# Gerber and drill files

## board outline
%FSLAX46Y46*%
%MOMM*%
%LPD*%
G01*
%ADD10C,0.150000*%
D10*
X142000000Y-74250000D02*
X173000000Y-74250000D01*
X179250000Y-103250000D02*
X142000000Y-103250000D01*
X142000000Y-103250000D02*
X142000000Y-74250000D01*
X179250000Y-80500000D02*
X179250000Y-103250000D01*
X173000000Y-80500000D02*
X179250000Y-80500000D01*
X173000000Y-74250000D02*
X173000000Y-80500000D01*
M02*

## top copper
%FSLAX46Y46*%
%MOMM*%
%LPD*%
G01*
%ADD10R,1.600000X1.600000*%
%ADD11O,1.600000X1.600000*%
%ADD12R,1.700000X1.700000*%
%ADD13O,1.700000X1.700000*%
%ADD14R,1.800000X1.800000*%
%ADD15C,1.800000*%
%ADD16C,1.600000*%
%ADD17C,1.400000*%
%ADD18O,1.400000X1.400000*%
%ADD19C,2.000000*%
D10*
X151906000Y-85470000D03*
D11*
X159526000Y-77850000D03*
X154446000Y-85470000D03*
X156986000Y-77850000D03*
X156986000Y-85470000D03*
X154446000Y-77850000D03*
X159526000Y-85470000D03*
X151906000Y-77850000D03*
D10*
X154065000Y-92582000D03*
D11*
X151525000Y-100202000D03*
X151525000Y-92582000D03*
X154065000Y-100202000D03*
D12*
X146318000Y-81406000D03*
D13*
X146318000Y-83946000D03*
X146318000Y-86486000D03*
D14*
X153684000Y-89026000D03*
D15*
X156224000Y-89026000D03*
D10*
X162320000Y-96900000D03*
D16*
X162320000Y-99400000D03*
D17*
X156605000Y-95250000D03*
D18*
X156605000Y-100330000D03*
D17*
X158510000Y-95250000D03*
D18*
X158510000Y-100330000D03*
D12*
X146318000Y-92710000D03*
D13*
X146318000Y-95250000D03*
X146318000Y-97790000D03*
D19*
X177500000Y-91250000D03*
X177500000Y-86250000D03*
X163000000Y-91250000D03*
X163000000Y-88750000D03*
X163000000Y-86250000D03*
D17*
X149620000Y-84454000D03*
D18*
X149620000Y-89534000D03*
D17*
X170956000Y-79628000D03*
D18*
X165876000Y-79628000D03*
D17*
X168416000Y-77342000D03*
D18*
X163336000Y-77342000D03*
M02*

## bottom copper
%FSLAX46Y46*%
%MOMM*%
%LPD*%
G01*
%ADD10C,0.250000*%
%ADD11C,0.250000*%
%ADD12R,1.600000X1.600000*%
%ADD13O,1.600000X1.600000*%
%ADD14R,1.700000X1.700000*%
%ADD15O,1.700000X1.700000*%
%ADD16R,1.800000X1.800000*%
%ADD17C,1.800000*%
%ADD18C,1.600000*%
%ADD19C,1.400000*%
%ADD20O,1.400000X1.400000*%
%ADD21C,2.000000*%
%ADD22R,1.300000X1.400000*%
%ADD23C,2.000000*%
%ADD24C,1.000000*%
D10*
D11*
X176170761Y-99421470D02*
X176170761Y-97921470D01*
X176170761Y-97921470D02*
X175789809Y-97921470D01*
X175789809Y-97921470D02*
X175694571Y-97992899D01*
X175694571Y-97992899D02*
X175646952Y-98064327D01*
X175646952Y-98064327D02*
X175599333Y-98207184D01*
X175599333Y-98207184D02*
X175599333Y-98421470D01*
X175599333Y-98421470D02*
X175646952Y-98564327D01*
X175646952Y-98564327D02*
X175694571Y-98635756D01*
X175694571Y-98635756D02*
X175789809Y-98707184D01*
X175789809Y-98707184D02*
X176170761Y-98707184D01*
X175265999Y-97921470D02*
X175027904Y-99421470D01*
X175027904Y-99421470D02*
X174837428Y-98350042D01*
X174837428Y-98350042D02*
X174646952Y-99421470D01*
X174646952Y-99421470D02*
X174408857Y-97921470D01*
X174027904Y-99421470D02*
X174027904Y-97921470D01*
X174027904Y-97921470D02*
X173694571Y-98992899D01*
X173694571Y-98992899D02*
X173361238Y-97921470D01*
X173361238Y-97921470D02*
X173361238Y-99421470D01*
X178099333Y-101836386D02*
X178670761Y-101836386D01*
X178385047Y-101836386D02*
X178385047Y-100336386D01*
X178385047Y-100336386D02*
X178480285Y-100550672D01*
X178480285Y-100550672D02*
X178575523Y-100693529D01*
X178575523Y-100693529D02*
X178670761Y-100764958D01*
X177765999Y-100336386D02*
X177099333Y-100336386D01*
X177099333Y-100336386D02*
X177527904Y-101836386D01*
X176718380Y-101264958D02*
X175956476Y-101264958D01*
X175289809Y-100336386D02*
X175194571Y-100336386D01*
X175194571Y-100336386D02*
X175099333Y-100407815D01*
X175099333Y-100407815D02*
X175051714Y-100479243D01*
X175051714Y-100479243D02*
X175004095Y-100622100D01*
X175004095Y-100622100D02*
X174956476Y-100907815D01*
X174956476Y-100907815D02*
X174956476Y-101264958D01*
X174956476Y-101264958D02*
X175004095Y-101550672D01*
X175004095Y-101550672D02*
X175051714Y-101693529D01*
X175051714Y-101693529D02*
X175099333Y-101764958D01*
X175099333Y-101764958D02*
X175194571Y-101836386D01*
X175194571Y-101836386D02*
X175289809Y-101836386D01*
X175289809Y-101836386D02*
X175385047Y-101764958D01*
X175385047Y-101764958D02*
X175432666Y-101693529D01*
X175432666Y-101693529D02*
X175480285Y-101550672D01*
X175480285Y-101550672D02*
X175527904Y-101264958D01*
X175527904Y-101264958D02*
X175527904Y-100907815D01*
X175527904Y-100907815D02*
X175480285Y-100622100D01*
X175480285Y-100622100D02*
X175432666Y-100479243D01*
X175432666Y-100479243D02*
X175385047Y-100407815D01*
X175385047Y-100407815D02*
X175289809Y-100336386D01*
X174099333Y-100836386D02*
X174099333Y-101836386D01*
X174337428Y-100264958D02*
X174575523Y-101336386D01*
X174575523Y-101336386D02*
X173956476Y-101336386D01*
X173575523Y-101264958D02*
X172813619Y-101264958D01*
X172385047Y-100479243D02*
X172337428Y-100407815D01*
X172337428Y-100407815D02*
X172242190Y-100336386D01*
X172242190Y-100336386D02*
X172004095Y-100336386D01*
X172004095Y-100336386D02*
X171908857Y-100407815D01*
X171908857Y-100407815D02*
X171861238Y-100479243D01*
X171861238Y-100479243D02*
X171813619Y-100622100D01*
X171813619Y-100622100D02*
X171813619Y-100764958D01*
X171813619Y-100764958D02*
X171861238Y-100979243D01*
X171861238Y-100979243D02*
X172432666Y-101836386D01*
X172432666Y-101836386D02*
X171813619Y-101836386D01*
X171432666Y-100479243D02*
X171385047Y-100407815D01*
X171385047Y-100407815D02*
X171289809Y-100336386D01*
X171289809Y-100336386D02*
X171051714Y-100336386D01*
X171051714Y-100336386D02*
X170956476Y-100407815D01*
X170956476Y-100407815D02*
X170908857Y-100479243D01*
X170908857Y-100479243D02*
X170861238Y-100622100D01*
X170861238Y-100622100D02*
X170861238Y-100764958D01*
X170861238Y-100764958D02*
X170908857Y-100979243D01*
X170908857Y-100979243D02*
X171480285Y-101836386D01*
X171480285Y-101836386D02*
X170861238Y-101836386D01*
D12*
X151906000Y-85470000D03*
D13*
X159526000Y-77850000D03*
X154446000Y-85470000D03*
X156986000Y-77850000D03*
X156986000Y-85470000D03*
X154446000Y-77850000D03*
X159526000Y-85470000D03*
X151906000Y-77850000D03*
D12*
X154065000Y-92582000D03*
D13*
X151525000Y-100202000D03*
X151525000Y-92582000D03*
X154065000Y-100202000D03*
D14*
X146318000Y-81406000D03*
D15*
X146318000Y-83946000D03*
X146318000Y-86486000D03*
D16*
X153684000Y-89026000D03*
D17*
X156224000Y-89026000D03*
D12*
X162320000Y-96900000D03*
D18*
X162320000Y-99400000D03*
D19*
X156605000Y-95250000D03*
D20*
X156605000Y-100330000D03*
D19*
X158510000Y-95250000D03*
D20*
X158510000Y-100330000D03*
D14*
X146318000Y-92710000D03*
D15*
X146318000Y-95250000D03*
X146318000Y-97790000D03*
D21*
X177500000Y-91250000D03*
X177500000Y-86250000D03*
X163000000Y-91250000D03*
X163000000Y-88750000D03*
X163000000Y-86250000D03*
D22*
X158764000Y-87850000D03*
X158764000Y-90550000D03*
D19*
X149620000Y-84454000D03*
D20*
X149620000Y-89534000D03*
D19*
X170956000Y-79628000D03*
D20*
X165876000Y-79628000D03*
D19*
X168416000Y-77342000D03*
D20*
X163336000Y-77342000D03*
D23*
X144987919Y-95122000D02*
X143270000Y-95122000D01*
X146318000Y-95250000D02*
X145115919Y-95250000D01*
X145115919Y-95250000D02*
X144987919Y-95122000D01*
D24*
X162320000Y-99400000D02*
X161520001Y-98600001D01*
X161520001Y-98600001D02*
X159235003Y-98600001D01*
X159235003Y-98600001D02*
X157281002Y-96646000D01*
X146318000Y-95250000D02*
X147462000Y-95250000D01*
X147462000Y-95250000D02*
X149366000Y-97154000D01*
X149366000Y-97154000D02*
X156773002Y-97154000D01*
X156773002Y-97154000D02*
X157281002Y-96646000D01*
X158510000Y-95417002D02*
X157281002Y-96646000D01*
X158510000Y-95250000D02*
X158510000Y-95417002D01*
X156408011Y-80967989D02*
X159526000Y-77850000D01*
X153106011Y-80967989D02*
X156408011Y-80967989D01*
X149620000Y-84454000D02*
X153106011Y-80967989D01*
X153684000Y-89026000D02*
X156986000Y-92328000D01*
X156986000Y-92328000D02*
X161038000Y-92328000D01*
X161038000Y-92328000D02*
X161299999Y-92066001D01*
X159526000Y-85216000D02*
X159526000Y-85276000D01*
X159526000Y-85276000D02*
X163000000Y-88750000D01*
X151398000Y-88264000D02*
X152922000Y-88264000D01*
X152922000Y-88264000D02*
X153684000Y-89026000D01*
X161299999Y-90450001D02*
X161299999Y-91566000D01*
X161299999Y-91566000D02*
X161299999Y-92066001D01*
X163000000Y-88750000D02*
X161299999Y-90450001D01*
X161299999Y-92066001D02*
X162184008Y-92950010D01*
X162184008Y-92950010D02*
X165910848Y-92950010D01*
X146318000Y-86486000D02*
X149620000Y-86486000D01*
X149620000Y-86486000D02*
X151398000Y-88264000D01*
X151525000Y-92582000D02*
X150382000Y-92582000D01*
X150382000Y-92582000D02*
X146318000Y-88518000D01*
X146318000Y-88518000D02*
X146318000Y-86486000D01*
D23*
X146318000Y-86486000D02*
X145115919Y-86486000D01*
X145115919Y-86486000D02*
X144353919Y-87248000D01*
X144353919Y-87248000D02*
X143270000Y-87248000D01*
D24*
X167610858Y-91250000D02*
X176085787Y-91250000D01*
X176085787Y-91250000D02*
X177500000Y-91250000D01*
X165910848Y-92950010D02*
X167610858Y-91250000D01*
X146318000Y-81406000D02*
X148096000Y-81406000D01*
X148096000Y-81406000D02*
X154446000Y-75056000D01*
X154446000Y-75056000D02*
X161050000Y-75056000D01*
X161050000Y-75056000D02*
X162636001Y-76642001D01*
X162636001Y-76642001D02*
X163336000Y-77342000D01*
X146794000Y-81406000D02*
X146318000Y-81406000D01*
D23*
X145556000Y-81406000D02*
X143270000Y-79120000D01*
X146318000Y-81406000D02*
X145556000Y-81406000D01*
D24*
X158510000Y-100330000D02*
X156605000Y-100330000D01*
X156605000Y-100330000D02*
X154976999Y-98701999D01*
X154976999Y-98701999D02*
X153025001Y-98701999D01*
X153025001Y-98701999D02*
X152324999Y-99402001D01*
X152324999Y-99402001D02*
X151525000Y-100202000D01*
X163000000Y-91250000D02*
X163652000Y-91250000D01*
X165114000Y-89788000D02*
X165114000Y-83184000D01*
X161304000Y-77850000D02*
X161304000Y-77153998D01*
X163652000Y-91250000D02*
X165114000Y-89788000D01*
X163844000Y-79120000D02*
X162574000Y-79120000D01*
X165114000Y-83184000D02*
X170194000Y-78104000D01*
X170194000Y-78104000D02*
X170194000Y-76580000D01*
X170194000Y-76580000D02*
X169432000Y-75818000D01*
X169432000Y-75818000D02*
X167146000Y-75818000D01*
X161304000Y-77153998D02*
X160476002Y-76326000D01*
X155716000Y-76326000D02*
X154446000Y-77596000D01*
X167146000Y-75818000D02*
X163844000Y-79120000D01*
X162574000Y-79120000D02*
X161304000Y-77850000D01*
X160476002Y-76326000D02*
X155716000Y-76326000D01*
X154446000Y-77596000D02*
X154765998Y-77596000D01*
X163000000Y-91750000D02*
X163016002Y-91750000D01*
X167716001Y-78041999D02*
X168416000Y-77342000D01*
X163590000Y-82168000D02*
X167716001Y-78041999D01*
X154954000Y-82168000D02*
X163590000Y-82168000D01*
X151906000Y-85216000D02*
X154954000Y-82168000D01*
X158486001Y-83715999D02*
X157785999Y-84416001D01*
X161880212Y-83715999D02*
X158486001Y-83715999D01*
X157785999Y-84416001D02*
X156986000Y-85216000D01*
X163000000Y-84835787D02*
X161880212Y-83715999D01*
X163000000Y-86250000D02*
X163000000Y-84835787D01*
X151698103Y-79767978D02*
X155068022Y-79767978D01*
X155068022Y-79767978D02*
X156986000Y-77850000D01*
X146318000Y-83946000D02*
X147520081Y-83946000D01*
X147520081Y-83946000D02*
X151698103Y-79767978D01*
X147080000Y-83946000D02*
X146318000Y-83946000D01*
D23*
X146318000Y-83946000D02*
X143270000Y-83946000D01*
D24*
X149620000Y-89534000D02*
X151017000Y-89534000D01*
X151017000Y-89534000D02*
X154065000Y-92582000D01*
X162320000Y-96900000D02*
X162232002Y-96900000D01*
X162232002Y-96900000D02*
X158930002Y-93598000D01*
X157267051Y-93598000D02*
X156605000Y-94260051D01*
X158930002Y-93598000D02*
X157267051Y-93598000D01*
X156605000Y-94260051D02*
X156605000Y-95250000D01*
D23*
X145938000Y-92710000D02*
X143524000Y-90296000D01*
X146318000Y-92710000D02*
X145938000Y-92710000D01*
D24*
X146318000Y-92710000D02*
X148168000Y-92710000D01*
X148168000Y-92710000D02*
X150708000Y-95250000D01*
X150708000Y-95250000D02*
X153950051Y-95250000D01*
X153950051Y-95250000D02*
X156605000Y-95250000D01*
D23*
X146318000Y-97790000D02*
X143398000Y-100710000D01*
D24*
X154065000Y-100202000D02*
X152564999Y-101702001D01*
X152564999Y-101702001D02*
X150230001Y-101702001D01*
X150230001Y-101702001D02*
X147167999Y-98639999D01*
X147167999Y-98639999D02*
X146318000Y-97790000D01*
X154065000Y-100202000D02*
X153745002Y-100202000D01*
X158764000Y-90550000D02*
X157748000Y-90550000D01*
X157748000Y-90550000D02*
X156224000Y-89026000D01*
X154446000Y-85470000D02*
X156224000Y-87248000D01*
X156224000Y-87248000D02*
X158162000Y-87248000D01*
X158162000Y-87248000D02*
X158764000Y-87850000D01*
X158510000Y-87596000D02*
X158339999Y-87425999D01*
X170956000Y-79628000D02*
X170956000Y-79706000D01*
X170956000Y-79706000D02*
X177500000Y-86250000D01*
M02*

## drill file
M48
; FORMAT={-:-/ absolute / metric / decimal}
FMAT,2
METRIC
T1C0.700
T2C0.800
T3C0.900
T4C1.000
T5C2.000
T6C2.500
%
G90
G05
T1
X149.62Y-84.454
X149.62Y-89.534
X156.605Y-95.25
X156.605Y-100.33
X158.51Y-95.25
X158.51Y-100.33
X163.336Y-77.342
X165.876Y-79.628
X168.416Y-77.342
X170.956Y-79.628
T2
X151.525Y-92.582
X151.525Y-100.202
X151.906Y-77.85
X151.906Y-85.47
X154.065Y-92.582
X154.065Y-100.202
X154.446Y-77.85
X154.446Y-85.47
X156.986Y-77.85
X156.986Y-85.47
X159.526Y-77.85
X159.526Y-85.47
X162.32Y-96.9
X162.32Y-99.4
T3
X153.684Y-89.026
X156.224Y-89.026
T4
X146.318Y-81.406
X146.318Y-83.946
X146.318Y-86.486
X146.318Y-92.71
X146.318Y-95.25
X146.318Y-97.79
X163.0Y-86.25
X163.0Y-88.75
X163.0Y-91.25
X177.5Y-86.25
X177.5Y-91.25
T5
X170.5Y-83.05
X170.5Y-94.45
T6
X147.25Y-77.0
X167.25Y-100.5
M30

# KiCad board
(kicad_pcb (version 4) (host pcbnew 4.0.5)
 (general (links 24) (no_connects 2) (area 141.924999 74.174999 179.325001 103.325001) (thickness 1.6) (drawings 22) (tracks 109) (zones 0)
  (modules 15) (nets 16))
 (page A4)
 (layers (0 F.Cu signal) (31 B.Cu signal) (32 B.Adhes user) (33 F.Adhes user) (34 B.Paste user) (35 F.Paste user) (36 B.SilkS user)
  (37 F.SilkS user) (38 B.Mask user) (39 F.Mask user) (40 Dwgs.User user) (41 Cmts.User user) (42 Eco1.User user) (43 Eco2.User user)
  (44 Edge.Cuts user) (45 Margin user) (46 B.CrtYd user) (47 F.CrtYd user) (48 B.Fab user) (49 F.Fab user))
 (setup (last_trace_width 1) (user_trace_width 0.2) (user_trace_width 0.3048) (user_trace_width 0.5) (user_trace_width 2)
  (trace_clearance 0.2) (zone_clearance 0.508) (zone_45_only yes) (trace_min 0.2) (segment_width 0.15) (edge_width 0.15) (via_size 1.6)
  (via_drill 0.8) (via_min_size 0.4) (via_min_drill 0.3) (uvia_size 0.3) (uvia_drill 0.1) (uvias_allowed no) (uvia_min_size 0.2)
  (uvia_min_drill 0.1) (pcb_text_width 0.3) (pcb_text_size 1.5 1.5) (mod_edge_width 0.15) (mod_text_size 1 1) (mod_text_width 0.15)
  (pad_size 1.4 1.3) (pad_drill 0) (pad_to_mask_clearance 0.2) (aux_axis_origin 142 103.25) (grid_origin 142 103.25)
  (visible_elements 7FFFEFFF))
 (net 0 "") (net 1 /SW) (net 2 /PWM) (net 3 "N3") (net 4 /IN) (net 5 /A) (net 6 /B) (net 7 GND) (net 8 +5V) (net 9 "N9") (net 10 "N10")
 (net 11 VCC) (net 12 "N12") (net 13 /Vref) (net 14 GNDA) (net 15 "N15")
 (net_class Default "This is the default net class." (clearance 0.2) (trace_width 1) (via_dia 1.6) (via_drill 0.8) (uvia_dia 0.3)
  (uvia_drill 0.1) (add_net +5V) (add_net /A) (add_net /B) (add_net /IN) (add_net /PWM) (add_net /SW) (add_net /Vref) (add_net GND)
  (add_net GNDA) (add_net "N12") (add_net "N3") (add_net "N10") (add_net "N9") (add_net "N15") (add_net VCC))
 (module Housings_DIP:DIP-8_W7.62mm (layer F.Cu) (at 151.906 85.47 90)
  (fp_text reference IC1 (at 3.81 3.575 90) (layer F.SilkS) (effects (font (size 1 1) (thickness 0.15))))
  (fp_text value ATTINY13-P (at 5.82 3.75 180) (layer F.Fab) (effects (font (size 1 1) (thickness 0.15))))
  (pad 1 thru_hole rect (at 0 0 90) (size 1.6 1.6) (drill 0.8) (layers *.Cu *.Mask) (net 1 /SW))
  (pad 5 thru_hole oval (at 7.62 7.62 90) (size 1.6 1.6) (drill 0.8) (layers *.Cu *.Mask) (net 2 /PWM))
  (pad 2 thru_hole oval (at 0 2.54 90) (size 1.6 1.6) (drill 0.8) (layers *.Cu *.Mask) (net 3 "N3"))
  (pad 6 thru_hole oval (at 7.62 5.08 90) (size 1.6 1.6) (drill 0.8) (layers *.Cu *.Mask) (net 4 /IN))
  (pad 3 thru_hole oval (at 0 5.08 90) (size 1.6 1.6) (drill 0.8) (layers *.Cu *.Mask) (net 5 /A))
  (pad 7 thru_hole oval (at 7.62 2.54 90) (size 1.6 1.6) (drill 0.8) (layers *.Cu *.Mask) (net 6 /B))
  (pad 4 thru_hole oval (at 0 7.62 90) (size 1.6 1.6) (drill 0.8) (layers *.Cu *.Mask) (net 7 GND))
  (pad 8 thru_hole oval (at 7.62 0 90) (size 1.6 1.6) (drill 0.8) (layers *.Cu *.Mask) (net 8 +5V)))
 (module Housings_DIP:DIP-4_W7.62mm (layer F.Cu) (at 154.065 92.582 270)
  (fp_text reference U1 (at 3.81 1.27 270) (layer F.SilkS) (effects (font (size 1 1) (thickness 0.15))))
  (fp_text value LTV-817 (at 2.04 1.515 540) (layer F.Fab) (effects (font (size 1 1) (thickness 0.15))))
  (pad 1 thru_hole rect (at 0 0 270) (size 1.6 1.6) (drill 0.8) (layers *.Cu *.Mask) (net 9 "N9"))
  (pad 3 thru_hole oval (at 7.62 2.54 270) (size 1.6 1.6) (drill 0.8) (layers *.Cu *.Mask) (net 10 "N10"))
  (pad 2 thru_hole oval (at 0 2.54 270) (size 1.6 1.6) (drill 0.8) (layers *.Cu *.Mask) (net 7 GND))
  (pad 4 thru_hole oval (at 7.62 0 270) (size 1.6 1.6) (drill 0.8) (layers *.Cu *.Mask) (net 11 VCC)))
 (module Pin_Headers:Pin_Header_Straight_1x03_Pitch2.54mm (layer F.Cu) (at 146.318 81.406)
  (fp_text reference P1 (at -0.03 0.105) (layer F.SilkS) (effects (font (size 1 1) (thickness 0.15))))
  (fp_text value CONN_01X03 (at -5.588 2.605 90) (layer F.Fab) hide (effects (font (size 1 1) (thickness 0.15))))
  (pad 1 thru_hole rect (at 0 0) (size 1.7 1.7) (drill 1) (layers *.Cu *.Mask) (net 8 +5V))
  (pad 2 thru_hole oval (at 0 2.54) (size 1.7 1.7) (drill 1) (layers *.Cu *.Mask) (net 4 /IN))
  (pad 3 thru_hole oval (at 0 5.08) (size 1.7 1.7) (drill 1) (layers *.Cu *.Mask) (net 7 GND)))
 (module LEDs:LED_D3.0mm (layer F.Cu) (at 153.684 89.026)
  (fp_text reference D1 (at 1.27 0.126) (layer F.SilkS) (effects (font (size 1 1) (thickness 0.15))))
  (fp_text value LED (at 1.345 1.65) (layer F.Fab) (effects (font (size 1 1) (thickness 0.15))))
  (pad 1 thru_hole rect (at 0 0) (size 1.8 1.8) (drill 0.9) (layers *.Cu *.Mask) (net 7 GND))
  (pad 2 thru_hole circle (at 2.54 0) (size 1.8 1.8) (drill 0.9) (layers *.Cu *.Mask) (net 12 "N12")))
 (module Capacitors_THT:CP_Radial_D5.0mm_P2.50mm (layer F.Cu) (at 162.32 96.9 270)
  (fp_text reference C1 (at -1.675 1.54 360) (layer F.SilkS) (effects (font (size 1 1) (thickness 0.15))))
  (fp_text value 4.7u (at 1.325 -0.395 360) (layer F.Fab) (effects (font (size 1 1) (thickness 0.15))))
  (pad 1 thru_hole rect (at 0 0 270) (size 1.6 1.6) (drill 0.8) (layers *.Cu *.Mask) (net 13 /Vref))
  (pad 2 thru_hole circle (at 2.5 0 270) (size 1.6 1.6) (drill 0.8) (layers *.Cu *.Mask) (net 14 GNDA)))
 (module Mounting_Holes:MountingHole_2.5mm (layer F.Cu) (at 147.25 77)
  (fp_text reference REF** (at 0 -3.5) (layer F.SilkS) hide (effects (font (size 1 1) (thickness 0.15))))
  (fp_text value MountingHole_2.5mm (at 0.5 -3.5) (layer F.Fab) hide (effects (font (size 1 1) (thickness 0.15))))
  (pad 1 np_thru_hole circle (at 0 0) (size 2.5 2.5) (drill 2.5) (layers *.Cu *.Mask)))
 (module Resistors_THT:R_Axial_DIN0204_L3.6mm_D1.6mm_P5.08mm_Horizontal (layer F.Cu) (at 156.605 95.25 270)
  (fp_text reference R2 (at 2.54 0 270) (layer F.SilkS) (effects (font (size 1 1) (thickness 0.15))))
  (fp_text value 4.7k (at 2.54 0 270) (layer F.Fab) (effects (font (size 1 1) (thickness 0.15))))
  (pad 1 thru_hole circle (at 0 0 270) (size 1.4 1.4) (drill 0.7) (layers *.Cu *.Mask) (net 13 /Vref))
  (pad 2 thru_hole oval (at 5.08 0 270) (size 1.4 1.4) (drill 0.7) (layers *.Cu *.Mask) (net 10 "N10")))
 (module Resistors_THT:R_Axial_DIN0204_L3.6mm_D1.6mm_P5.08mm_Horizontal (layer F.Cu) (at 158.51 95.25 270)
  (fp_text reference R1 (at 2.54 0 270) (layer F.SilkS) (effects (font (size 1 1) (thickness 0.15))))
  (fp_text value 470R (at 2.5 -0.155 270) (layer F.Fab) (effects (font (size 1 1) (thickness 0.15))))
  (pad 1 thru_hole circle (at 0 0 270) (size 1.4 1.4) (drill 0.7) (layers *.Cu *.Mask) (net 14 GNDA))
  (pad 2 thru_hole oval (at 5.08 0 270) (size 1.4 1.4) (drill 0.7) (layers *.Cu *.Mask) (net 10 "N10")))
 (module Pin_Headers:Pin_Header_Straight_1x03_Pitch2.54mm (layer F.Cu) (at 146.318 92.71)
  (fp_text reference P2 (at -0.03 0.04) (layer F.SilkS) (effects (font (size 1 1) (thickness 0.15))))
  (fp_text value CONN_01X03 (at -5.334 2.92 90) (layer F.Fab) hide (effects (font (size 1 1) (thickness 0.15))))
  (pad 1 thru_hole rect (at 0 0) (size 1.7 1.7) (drill 1) (layers *.Cu *.Mask) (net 13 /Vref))
  (pad 2 thru_hole oval (at 0 2.54) (size 1.7 1.7) (drill 1) (layers *.Cu *.Mask) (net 14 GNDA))
  (pad 3 thru_hole oval (at 0 5.08) (size 1.7 1.7) (drill 1) (layers *.Cu *.Mask) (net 11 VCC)))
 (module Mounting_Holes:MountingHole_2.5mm (layer F.Cu) (at 167.25 100.5)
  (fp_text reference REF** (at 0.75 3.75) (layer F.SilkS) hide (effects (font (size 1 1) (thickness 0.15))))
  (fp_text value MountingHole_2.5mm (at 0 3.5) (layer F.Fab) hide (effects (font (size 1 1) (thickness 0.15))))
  (pad 1 np_thru_hole circle (at 0 0) (size 2.5 2.5) (drill 2.5) (layers *.Cu *.Mask)))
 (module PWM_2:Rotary (layer F.Cu) (at 170.5 88.75 270)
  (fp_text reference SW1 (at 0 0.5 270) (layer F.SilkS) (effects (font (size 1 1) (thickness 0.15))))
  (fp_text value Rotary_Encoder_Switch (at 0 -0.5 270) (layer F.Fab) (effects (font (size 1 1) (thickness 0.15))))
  (pad 5 thru_hole circle (at 2.5 -7 270) (size 2 2) (drill 1) (layers *.Cu *.Mask) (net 7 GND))
  (pad 4 thru_hole circle (at -2.5 -7 270) (size 2 2) (drill 1) (layers *.Cu *.Mask) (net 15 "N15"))
  (pad 3 thru_hole circle (at 2.5 7.5 270) (size 2 2) (drill 1) (layers *.Cu *.Mask) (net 6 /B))
  (pad 2 thru_hole circle (at 0 7.5 270) (size 2 2) (drill 1) (layers *.Cu *.Mask) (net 7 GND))
  (pad 1 thru_hole circle (at -2.5 7.5 270) (size 2 2) (drill 1) (layers *.Cu *.Mask) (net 5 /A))
  (pad "" np_thru_hole circle (at -5.7 0 270) (size 2 2) (drill 2) (layers *.Cu *.Mask))
  (pad "" np_thru_hole circle (at 5.7 0 270) (size 2 2) (drill 2) (layers *.Cu *.Mask)))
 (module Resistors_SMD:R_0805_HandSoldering (layer B.Cu) (at 158.764 89.2 270)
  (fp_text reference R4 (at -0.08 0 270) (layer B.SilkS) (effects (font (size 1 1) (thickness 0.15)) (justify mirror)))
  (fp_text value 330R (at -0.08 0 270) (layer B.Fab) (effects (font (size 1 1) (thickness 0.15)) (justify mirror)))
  (pad 1 smd rect (at -1.35 0 270) (size 1.4 1.3) (layers B.Cu B.Paste B.Mask) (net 3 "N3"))
  (pad 2 smd rect (at 1.35 0 270) (size 1.4 1.3) (layers B.Cu B.Paste B.Mask) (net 12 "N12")))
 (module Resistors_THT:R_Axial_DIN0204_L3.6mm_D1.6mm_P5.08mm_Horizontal (layer F.Cu) (at 149.62 84.454 270)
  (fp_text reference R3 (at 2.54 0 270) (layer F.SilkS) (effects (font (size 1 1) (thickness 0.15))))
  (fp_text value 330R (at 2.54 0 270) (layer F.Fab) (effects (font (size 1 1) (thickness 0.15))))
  (pad 1 thru_hole circle (at 0 0 270) (size 1.4 1.4) (drill 0.7) (layers *.Cu *.Mask) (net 2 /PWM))
  (pad 2 thru_hole oval (at 5.08 0 270) (size 1.4 1.4) (drill 0.7) (layers *.Cu *.Mask) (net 9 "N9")))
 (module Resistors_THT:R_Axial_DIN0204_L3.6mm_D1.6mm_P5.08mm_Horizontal (layer F.Cu) (at 170.956 79.628 180)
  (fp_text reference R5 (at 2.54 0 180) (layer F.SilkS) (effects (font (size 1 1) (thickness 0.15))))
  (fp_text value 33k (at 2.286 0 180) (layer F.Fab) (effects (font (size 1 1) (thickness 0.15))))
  (pad 1 thru_hole circle (at 0 0 180) (size 1.4 1.4) (drill 0.7) (layers *.Cu *.Mask) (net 15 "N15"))
  (pad 2 thru_hole oval (at 5.08 0 180) (size 1.4 1.4) (drill 0.7) (layers *.Cu *.Mask) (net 1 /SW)))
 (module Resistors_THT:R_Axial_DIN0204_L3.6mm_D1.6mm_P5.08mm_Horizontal (layer F.Cu) (at 168.416 77.342 180)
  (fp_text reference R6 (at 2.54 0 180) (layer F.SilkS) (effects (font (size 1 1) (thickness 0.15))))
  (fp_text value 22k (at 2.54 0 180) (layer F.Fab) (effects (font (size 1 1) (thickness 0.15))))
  (pad 1 thru_hole circle (at 0 0 180) (size 1.4 1.4) (drill 0.7) (layers *.Cu *.Mask) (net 1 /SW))
  (pad 2 thru_hole oval (at 5.08 0 180) (size 1.4 1.4) (drill 0.7) (layers *.Cu *.Mask) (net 8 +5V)))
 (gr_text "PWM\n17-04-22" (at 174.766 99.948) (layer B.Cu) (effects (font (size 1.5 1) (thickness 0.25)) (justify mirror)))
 (gr_line (start 142 74.25) (end 173 74.25) (layer Edge.Cuts) (width 0.15))
 (gr_line (start 179.25 103.25) (end 142 103.25) (layer Edge.Cuts) (width 0.15))
 (gr_line (start 142 103.25) (end 142 74.25) (angle 90) (layer Edge.Cuts) (width 0.15))
 (gr_line (start 179.25 80.5) (end 179.25 103.25) (angle 90) (layer Edge.Cuts) (width 0.15))
 (gr_line (start 173 80.5) (end 179.25 80.5) (angle 90) (layer Edge.Cuts) (width 0.15))
 (gr_line (start 173 74.25) (end 173 80.5) (angle 90) (layer Edge.Cuts) (width 0.15))
 (segment (start 144.987919 95.122) (end 143.27 95.122) (width 2) (layer B.Cu) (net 14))
 (segment (start 146.318 95.25) (end 145.115919 95.25) (width 2) (layer B.Cu) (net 14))
 (segment (start 145.115919 95.25) (end 144.987919 95.122) (width 2) (layer B.Cu) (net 14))
 (segment (start 162.32 99.4) (end 161.520001 98.600001) (width 1) (layer B.Cu) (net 14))
 (segment (start 161.520001 98.600001) (end 159.235003 98.600001) (width 1) (layer B.Cu) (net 14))
 (segment (start 159.235003 98.600001) (end 157.281002 96.646) (width 1) (layer B.Cu) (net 14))
 (segment (start 146.318 95.25) (end 147.462 95.25) (width 1) (layer B.Cu) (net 14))
 (segment (start 147.462 95.25) (end 149.366 97.154) (width 1) (layer B.Cu) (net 14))
 (segment (start 149.366 97.154) (end 156.773002 97.154) (width 1) (layer B.Cu) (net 14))
 (segment (start 156.773002 97.154) (end 157.281002 96.646) (width 1) (layer B.Cu) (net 14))
 (segment (start 158.51 95.417002) (end 157.281002 96.646) (width 1) (layer B.Cu) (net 14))
 (segment (start 158.51 95.25) (end 158.51 95.417002) (width 1) (layer B.Cu) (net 14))
 (segment (start 156.408011 80.967989) (end 159.526 77.85) (width 1) (layer B.Cu) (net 2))
 (segment (start 153.106011 80.967989) (end 156.408011 80.967989) (width 1) (layer B.Cu) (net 2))
 (segment (start 149.62 84.454) (end 153.106011 80.967989) (width 1) (layer B.Cu) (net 2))
 (segment (start 153.684 89.026) (end 156.986 92.328) (width 1) (layer B.Cu) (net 7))
 (segment (start 156.986 92.328) (end 161.038 92.328) (width 1) (layer B.Cu) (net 7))
 (segment (start 161.038 92.328) (end 161.299999 92.066001) (width 1) (layer B.Cu) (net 7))
 (segment (start 159.526 85.216) (end 159.526 85.276) (width 1) (layer B.Cu) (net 7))
 (segment (start 159.526 85.276) (end 163 88.75) (width 1) (layer B.Cu) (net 7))
 (segment (start 151.398 88.264) (end 152.922 88.264) (width 1) (layer B.Cu) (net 7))
 (segment (start 152.922 88.264) (end 153.684 89.026) (width 1) (layer B.Cu) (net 7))
 (segment (start 161.299999 90.450001) (end 161.299999 91.566) (width 1) (layer B.Cu) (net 7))
 (segment (start 161.299999 91.566) (end 161.299999 92.066001) (width 1) (layer B.Cu) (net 7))
 (segment (start 163 88.75) (end 161.299999 90.450001) (width 1) (layer B.Cu) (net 7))
 (segment (start 161.299999 92.066001) (end 162.184008 92.95001) (width 1) (layer B.Cu) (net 7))
 (segment (start 162.184008 92.95001) (end 165.910848 92.95001) (width 1) (layer B.Cu) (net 7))
 (segment (start 146.318 86.486) (end 149.62 86.486) (width 1) (layer B.Cu) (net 7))
 (segment (start 149.62 86.486) (end 151.398 88.264) (width 1) (layer B.Cu) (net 7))
 (segment (start 151.525 92.582) (end 150.382 92.582) (width 1) (layer B.Cu) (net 7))
 (segment (start 150.382 92.582) (end 146.318 88.518) (width 1) (layer B.Cu) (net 7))
 (segment (start 146.318 88.518) (end 146.318 86.486) (width 1) (layer B.Cu) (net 7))
 (segment (start 146.318 86.486) (end 145.115919 86.486) (width 2) (layer B.Cu) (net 7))
 (segment (start 145.115919 86.486) (end 144.353919 87.248) (width 2) (layer B.Cu) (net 7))
 (segment (start 144.353919 87.248) (end 143.27 87.248) (width 2) (layer B.Cu) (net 7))
 (segment (start 167.610858 91.25) (end 176.085787 91.25) (width 1) (layer B.Cu) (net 7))
 (segment (start 176.085787 91.25) (end 177.5 91.25) (width 1) (layer B.Cu) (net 7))
 (segment (start 165.910848 92.95001) (end 167.610858 91.25) (width 1) (layer B.Cu) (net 7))
 (segment (start 146.318 81.406) (end 148.096 81.406) (width 1) (layer B.Cu) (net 8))
 (segment (start 148.096 81.406) (end 154.446 75.056) (width 1) (layer B.Cu) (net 8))
 (segment (start 154.446 75.056) (end 161.05 75.056) (width 1) (layer B.Cu) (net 8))
 (segment (start 161.05 75.056) (end 162.636001 76.642001) (width 1) (layer B.Cu) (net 8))
 (segment (start 162.636001 76.642001) (end 163.336 77.342) (width 1) (layer B.Cu) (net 8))
 (segment (start 146.794 81.406) (end 146.318 81.406) (width 1) (layer B.Cu) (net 8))
 (segment (start 145.556 81.406) (end 143.27 79.12) (width 2) (layer B.Cu) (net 8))
 (segment (start 146.318 81.406) (end 145.556 81.406) (width 2) (layer B.Cu) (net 8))
 (segment (start 158.51 100.33) (end 156.605 100.33) (width 1) (layer B.Cu) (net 10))
 (segment (start 156.605 100.33) (end 154.976999 98.701999) (width 1) (layer B.Cu) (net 10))
 (segment (start 154.976999 98.701999) (end 153.025001 98.701999) (width 1) (layer B.Cu) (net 10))
 (segment (start 153.025001 98.701999) (end 152.324999 99.402001) (width 1) (layer B.Cu) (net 10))
 (segment (start 152.324999 99.402001) (end 151.525 100.202) (width 1) (layer B.Cu) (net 10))
 (segment (start 163 91.25) (end 163.652 91.25) (width 1) (layer B.Cu) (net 6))
 (segment (start 165.114 89.788) (end 165.114 83.184) (width 1) (layer B.Cu) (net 6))
 (segment (start 161.304 77.85) (end 161.304 77.153998) (width 1) (layer B.Cu) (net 6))
 (segment (start 163.652 91.25) (end 165.114 89.788) (width 1) (layer B.Cu) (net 6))
 (segment (start 163.844 79.12) (end 162.574 79.12) (width 1) (layer B.Cu) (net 6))
 (segment (start 165.114 83.184) (end 170.194 78.104) (width 1) (layer B.Cu) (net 6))
 (segment (start 170.194 78.104) (end 170.194 76.58) (width 1) (layer B.Cu) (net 6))
 (segment (start 170.194 76.58) (end 169.432 75.818) (width 1) (layer B.Cu) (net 6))
 (segment (start 169.432 75.818) (end 167.146 75.818) (width 1) (layer B.Cu) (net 6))
 (segment (start 161.304 77.153998) (end 160.476002 76.326) (width 1) (layer B.Cu) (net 6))
 (segment (start 155.716 76.326) (end 154.446 77.596) (width 1) (layer B.Cu) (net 6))
 (segment (start 167.146 75.818) (end 163.844 79.12) (width 1) (layer B.Cu) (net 6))
 (segment (start 162.574 79.12) (end 161.304 77.85) (width 1) (layer B.Cu) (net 6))
 (segment (start 160.476002 76.326) (end 155.716 76.326) (width 1) (layer B.Cu) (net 6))
 (segment (start 154.446 77.596) (end 154.765998 77.596) (width 1) (layer B.Cu) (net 6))
 (segment (start 163 91.75) (end 163.016002 91.75) (width 1) (layer B.Cu) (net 6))
 (segment (start 167.716001 78.041999) (end 168.416 77.342) (width 1) (layer B.Cu) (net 1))
 (segment (start 163.59 82.168) (end 167.716001 78.041999) (width 1) (layer B.Cu) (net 1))
 (segment (start 154.954 82.168) (end 163.59 82.168) (width 1) (layer B.Cu) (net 1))
 (segment (start 151.906 85.216) (end 154.954 82.168) (width 1) (layer B.Cu) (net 1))
 (segment (start 158.486001 83.715999) (end 157.785999 84.416001) (width 1) (layer B.Cu) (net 5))
 (segment (start 161.880212 83.715999) (end 158.486001 83.715999) (width 1) (layer B.Cu) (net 5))
 (segment (start 157.785999 84.416001) (end 156.986 85.216) (width 1) (layer B.Cu) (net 5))
 (segment (start 163 84.835787) (end 161.880212 83.715999) (width 1) (layer B.Cu) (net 5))
 (segment (start 163 86.25) (end 163 84.835787) (width 1) (layer B.Cu) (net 5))
 (segment (start 151.698103 79.767978) (end 155.068022 79.767978) (width 1) (layer B.Cu) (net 4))
 (segment (start 155.068022 79.767978) (end 156.986 77.85) (width 1) (layer B.Cu) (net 4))
 (segment (start 146.318 83.946) (end 147.520081 83.946) (width 1) (layer B.Cu) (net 4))
 (segment (start 147.520081 83.946) (end 151.698103 79.767978) (width 1) (layer B.Cu) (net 4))
 (segment (start 147.08 83.946) (end 146.318 83.946) (width 1) (layer B.Cu) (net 4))
 (segment (start 146.318 83.946) (end 143.27 83.946) (width 2) (layer B.Cu) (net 4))
 (segment (start 149.62 89.534) (end 151.017 89.534) (width 1) (layer B.Cu) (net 9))
 (segment (start 151.017 89.534) (end 154.065 92.582) (width 1) (layer B.Cu) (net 9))
 (segment (start 162.32 96.9) (end 162.232002 96.9) (width 1) (layer B.Cu) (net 13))
 (segment (start 162.232002 96.9) (end 158.930002 93.598) (width 1) (layer B.Cu) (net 13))
 (segment (start 157.267051 93.598) (end 156.605 94.260051) (width 1) (layer B.Cu) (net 13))
 (segment (start 158.930002 93.598) (end 157.267051 93.598) (width 1) (layer B.Cu) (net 13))
 (segment (start 156.605 94.260051) (end 156.605 95.25) (width 1) (layer B.Cu) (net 13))
 (segment (start 145.938 92.71) (end 143.524 90.296) (width 2) (layer B.Cu) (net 13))
 (segment (start 146.318 92.71) (end 145.938 92.71) (width 2) (layer B.Cu) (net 13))
 (segment (start 146.318 92.71) (end 148.168 92.71) (width 1) (layer B.Cu) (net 13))
 (segment (start 148.168 92.71) (end 150.708 95.25) (width 1) (layer B.Cu) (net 13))
 (segment (start 150.708 95.25) (end 153.950051 95.25) (width 1) (layer B.Cu) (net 13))
 (segment (start 153.950051 95.25) (end 156.605 95.25) (width 1) (layer B.Cu) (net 13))
 (segment (start 146.318 97.79) (end 143.398 100.71) (width 2) (layer B.Cu) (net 11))
 (segment (start 154.065 100.202) (end 152.564999 101.702001) (width 1) (layer B.Cu) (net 11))
 (segment (start 152.564999 101.702001) (end 150.230001 101.702001) (width 1) (layer B.Cu) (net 11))
 (segment (start 150.230001 101.702001) (end 147.167999 98.639999) (width 1) (layer B.Cu) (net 11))
 (segment (start 147.167999 98.639999) (end 146.318 97.79) (width 1) (layer B.Cu) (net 11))
 (segment (start 154.065 100.202) (end 153.745002 100.202) (width 1) (layer B.Cu) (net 11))
 (segment (start 158.764 90.55) (end 157.748 90.55) (width 1) (layer B.Cu) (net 12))
 (segment (start 157.748 90.55) (end 156.224 89.026) (width 1) (layer B.Cu) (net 12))
 (segment (start 154.446 85.47) (end 156.224 87.248) (width 1) (layer B.Cu) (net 3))
 (segment (start 156.224 87.248) (end 158.162 87.248) (width 1) (layer B.Cu) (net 3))
 (segment (start 158.162 87.248) (end 158.764 87.85) (width 1) (layer B.Cu) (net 3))
 (segment (start 158.51 87.596) (end 158.339999 87.425999) (width 1) (layer B.Cu) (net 3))
 (segment (start 170.956 79.628) (end 170.956 79.706) (width 1) (layer B.Cu) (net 15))
 (segment (start 170.956 79.706) (end 177.5 86.25) (width 1) (layer B.Cu) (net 15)))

